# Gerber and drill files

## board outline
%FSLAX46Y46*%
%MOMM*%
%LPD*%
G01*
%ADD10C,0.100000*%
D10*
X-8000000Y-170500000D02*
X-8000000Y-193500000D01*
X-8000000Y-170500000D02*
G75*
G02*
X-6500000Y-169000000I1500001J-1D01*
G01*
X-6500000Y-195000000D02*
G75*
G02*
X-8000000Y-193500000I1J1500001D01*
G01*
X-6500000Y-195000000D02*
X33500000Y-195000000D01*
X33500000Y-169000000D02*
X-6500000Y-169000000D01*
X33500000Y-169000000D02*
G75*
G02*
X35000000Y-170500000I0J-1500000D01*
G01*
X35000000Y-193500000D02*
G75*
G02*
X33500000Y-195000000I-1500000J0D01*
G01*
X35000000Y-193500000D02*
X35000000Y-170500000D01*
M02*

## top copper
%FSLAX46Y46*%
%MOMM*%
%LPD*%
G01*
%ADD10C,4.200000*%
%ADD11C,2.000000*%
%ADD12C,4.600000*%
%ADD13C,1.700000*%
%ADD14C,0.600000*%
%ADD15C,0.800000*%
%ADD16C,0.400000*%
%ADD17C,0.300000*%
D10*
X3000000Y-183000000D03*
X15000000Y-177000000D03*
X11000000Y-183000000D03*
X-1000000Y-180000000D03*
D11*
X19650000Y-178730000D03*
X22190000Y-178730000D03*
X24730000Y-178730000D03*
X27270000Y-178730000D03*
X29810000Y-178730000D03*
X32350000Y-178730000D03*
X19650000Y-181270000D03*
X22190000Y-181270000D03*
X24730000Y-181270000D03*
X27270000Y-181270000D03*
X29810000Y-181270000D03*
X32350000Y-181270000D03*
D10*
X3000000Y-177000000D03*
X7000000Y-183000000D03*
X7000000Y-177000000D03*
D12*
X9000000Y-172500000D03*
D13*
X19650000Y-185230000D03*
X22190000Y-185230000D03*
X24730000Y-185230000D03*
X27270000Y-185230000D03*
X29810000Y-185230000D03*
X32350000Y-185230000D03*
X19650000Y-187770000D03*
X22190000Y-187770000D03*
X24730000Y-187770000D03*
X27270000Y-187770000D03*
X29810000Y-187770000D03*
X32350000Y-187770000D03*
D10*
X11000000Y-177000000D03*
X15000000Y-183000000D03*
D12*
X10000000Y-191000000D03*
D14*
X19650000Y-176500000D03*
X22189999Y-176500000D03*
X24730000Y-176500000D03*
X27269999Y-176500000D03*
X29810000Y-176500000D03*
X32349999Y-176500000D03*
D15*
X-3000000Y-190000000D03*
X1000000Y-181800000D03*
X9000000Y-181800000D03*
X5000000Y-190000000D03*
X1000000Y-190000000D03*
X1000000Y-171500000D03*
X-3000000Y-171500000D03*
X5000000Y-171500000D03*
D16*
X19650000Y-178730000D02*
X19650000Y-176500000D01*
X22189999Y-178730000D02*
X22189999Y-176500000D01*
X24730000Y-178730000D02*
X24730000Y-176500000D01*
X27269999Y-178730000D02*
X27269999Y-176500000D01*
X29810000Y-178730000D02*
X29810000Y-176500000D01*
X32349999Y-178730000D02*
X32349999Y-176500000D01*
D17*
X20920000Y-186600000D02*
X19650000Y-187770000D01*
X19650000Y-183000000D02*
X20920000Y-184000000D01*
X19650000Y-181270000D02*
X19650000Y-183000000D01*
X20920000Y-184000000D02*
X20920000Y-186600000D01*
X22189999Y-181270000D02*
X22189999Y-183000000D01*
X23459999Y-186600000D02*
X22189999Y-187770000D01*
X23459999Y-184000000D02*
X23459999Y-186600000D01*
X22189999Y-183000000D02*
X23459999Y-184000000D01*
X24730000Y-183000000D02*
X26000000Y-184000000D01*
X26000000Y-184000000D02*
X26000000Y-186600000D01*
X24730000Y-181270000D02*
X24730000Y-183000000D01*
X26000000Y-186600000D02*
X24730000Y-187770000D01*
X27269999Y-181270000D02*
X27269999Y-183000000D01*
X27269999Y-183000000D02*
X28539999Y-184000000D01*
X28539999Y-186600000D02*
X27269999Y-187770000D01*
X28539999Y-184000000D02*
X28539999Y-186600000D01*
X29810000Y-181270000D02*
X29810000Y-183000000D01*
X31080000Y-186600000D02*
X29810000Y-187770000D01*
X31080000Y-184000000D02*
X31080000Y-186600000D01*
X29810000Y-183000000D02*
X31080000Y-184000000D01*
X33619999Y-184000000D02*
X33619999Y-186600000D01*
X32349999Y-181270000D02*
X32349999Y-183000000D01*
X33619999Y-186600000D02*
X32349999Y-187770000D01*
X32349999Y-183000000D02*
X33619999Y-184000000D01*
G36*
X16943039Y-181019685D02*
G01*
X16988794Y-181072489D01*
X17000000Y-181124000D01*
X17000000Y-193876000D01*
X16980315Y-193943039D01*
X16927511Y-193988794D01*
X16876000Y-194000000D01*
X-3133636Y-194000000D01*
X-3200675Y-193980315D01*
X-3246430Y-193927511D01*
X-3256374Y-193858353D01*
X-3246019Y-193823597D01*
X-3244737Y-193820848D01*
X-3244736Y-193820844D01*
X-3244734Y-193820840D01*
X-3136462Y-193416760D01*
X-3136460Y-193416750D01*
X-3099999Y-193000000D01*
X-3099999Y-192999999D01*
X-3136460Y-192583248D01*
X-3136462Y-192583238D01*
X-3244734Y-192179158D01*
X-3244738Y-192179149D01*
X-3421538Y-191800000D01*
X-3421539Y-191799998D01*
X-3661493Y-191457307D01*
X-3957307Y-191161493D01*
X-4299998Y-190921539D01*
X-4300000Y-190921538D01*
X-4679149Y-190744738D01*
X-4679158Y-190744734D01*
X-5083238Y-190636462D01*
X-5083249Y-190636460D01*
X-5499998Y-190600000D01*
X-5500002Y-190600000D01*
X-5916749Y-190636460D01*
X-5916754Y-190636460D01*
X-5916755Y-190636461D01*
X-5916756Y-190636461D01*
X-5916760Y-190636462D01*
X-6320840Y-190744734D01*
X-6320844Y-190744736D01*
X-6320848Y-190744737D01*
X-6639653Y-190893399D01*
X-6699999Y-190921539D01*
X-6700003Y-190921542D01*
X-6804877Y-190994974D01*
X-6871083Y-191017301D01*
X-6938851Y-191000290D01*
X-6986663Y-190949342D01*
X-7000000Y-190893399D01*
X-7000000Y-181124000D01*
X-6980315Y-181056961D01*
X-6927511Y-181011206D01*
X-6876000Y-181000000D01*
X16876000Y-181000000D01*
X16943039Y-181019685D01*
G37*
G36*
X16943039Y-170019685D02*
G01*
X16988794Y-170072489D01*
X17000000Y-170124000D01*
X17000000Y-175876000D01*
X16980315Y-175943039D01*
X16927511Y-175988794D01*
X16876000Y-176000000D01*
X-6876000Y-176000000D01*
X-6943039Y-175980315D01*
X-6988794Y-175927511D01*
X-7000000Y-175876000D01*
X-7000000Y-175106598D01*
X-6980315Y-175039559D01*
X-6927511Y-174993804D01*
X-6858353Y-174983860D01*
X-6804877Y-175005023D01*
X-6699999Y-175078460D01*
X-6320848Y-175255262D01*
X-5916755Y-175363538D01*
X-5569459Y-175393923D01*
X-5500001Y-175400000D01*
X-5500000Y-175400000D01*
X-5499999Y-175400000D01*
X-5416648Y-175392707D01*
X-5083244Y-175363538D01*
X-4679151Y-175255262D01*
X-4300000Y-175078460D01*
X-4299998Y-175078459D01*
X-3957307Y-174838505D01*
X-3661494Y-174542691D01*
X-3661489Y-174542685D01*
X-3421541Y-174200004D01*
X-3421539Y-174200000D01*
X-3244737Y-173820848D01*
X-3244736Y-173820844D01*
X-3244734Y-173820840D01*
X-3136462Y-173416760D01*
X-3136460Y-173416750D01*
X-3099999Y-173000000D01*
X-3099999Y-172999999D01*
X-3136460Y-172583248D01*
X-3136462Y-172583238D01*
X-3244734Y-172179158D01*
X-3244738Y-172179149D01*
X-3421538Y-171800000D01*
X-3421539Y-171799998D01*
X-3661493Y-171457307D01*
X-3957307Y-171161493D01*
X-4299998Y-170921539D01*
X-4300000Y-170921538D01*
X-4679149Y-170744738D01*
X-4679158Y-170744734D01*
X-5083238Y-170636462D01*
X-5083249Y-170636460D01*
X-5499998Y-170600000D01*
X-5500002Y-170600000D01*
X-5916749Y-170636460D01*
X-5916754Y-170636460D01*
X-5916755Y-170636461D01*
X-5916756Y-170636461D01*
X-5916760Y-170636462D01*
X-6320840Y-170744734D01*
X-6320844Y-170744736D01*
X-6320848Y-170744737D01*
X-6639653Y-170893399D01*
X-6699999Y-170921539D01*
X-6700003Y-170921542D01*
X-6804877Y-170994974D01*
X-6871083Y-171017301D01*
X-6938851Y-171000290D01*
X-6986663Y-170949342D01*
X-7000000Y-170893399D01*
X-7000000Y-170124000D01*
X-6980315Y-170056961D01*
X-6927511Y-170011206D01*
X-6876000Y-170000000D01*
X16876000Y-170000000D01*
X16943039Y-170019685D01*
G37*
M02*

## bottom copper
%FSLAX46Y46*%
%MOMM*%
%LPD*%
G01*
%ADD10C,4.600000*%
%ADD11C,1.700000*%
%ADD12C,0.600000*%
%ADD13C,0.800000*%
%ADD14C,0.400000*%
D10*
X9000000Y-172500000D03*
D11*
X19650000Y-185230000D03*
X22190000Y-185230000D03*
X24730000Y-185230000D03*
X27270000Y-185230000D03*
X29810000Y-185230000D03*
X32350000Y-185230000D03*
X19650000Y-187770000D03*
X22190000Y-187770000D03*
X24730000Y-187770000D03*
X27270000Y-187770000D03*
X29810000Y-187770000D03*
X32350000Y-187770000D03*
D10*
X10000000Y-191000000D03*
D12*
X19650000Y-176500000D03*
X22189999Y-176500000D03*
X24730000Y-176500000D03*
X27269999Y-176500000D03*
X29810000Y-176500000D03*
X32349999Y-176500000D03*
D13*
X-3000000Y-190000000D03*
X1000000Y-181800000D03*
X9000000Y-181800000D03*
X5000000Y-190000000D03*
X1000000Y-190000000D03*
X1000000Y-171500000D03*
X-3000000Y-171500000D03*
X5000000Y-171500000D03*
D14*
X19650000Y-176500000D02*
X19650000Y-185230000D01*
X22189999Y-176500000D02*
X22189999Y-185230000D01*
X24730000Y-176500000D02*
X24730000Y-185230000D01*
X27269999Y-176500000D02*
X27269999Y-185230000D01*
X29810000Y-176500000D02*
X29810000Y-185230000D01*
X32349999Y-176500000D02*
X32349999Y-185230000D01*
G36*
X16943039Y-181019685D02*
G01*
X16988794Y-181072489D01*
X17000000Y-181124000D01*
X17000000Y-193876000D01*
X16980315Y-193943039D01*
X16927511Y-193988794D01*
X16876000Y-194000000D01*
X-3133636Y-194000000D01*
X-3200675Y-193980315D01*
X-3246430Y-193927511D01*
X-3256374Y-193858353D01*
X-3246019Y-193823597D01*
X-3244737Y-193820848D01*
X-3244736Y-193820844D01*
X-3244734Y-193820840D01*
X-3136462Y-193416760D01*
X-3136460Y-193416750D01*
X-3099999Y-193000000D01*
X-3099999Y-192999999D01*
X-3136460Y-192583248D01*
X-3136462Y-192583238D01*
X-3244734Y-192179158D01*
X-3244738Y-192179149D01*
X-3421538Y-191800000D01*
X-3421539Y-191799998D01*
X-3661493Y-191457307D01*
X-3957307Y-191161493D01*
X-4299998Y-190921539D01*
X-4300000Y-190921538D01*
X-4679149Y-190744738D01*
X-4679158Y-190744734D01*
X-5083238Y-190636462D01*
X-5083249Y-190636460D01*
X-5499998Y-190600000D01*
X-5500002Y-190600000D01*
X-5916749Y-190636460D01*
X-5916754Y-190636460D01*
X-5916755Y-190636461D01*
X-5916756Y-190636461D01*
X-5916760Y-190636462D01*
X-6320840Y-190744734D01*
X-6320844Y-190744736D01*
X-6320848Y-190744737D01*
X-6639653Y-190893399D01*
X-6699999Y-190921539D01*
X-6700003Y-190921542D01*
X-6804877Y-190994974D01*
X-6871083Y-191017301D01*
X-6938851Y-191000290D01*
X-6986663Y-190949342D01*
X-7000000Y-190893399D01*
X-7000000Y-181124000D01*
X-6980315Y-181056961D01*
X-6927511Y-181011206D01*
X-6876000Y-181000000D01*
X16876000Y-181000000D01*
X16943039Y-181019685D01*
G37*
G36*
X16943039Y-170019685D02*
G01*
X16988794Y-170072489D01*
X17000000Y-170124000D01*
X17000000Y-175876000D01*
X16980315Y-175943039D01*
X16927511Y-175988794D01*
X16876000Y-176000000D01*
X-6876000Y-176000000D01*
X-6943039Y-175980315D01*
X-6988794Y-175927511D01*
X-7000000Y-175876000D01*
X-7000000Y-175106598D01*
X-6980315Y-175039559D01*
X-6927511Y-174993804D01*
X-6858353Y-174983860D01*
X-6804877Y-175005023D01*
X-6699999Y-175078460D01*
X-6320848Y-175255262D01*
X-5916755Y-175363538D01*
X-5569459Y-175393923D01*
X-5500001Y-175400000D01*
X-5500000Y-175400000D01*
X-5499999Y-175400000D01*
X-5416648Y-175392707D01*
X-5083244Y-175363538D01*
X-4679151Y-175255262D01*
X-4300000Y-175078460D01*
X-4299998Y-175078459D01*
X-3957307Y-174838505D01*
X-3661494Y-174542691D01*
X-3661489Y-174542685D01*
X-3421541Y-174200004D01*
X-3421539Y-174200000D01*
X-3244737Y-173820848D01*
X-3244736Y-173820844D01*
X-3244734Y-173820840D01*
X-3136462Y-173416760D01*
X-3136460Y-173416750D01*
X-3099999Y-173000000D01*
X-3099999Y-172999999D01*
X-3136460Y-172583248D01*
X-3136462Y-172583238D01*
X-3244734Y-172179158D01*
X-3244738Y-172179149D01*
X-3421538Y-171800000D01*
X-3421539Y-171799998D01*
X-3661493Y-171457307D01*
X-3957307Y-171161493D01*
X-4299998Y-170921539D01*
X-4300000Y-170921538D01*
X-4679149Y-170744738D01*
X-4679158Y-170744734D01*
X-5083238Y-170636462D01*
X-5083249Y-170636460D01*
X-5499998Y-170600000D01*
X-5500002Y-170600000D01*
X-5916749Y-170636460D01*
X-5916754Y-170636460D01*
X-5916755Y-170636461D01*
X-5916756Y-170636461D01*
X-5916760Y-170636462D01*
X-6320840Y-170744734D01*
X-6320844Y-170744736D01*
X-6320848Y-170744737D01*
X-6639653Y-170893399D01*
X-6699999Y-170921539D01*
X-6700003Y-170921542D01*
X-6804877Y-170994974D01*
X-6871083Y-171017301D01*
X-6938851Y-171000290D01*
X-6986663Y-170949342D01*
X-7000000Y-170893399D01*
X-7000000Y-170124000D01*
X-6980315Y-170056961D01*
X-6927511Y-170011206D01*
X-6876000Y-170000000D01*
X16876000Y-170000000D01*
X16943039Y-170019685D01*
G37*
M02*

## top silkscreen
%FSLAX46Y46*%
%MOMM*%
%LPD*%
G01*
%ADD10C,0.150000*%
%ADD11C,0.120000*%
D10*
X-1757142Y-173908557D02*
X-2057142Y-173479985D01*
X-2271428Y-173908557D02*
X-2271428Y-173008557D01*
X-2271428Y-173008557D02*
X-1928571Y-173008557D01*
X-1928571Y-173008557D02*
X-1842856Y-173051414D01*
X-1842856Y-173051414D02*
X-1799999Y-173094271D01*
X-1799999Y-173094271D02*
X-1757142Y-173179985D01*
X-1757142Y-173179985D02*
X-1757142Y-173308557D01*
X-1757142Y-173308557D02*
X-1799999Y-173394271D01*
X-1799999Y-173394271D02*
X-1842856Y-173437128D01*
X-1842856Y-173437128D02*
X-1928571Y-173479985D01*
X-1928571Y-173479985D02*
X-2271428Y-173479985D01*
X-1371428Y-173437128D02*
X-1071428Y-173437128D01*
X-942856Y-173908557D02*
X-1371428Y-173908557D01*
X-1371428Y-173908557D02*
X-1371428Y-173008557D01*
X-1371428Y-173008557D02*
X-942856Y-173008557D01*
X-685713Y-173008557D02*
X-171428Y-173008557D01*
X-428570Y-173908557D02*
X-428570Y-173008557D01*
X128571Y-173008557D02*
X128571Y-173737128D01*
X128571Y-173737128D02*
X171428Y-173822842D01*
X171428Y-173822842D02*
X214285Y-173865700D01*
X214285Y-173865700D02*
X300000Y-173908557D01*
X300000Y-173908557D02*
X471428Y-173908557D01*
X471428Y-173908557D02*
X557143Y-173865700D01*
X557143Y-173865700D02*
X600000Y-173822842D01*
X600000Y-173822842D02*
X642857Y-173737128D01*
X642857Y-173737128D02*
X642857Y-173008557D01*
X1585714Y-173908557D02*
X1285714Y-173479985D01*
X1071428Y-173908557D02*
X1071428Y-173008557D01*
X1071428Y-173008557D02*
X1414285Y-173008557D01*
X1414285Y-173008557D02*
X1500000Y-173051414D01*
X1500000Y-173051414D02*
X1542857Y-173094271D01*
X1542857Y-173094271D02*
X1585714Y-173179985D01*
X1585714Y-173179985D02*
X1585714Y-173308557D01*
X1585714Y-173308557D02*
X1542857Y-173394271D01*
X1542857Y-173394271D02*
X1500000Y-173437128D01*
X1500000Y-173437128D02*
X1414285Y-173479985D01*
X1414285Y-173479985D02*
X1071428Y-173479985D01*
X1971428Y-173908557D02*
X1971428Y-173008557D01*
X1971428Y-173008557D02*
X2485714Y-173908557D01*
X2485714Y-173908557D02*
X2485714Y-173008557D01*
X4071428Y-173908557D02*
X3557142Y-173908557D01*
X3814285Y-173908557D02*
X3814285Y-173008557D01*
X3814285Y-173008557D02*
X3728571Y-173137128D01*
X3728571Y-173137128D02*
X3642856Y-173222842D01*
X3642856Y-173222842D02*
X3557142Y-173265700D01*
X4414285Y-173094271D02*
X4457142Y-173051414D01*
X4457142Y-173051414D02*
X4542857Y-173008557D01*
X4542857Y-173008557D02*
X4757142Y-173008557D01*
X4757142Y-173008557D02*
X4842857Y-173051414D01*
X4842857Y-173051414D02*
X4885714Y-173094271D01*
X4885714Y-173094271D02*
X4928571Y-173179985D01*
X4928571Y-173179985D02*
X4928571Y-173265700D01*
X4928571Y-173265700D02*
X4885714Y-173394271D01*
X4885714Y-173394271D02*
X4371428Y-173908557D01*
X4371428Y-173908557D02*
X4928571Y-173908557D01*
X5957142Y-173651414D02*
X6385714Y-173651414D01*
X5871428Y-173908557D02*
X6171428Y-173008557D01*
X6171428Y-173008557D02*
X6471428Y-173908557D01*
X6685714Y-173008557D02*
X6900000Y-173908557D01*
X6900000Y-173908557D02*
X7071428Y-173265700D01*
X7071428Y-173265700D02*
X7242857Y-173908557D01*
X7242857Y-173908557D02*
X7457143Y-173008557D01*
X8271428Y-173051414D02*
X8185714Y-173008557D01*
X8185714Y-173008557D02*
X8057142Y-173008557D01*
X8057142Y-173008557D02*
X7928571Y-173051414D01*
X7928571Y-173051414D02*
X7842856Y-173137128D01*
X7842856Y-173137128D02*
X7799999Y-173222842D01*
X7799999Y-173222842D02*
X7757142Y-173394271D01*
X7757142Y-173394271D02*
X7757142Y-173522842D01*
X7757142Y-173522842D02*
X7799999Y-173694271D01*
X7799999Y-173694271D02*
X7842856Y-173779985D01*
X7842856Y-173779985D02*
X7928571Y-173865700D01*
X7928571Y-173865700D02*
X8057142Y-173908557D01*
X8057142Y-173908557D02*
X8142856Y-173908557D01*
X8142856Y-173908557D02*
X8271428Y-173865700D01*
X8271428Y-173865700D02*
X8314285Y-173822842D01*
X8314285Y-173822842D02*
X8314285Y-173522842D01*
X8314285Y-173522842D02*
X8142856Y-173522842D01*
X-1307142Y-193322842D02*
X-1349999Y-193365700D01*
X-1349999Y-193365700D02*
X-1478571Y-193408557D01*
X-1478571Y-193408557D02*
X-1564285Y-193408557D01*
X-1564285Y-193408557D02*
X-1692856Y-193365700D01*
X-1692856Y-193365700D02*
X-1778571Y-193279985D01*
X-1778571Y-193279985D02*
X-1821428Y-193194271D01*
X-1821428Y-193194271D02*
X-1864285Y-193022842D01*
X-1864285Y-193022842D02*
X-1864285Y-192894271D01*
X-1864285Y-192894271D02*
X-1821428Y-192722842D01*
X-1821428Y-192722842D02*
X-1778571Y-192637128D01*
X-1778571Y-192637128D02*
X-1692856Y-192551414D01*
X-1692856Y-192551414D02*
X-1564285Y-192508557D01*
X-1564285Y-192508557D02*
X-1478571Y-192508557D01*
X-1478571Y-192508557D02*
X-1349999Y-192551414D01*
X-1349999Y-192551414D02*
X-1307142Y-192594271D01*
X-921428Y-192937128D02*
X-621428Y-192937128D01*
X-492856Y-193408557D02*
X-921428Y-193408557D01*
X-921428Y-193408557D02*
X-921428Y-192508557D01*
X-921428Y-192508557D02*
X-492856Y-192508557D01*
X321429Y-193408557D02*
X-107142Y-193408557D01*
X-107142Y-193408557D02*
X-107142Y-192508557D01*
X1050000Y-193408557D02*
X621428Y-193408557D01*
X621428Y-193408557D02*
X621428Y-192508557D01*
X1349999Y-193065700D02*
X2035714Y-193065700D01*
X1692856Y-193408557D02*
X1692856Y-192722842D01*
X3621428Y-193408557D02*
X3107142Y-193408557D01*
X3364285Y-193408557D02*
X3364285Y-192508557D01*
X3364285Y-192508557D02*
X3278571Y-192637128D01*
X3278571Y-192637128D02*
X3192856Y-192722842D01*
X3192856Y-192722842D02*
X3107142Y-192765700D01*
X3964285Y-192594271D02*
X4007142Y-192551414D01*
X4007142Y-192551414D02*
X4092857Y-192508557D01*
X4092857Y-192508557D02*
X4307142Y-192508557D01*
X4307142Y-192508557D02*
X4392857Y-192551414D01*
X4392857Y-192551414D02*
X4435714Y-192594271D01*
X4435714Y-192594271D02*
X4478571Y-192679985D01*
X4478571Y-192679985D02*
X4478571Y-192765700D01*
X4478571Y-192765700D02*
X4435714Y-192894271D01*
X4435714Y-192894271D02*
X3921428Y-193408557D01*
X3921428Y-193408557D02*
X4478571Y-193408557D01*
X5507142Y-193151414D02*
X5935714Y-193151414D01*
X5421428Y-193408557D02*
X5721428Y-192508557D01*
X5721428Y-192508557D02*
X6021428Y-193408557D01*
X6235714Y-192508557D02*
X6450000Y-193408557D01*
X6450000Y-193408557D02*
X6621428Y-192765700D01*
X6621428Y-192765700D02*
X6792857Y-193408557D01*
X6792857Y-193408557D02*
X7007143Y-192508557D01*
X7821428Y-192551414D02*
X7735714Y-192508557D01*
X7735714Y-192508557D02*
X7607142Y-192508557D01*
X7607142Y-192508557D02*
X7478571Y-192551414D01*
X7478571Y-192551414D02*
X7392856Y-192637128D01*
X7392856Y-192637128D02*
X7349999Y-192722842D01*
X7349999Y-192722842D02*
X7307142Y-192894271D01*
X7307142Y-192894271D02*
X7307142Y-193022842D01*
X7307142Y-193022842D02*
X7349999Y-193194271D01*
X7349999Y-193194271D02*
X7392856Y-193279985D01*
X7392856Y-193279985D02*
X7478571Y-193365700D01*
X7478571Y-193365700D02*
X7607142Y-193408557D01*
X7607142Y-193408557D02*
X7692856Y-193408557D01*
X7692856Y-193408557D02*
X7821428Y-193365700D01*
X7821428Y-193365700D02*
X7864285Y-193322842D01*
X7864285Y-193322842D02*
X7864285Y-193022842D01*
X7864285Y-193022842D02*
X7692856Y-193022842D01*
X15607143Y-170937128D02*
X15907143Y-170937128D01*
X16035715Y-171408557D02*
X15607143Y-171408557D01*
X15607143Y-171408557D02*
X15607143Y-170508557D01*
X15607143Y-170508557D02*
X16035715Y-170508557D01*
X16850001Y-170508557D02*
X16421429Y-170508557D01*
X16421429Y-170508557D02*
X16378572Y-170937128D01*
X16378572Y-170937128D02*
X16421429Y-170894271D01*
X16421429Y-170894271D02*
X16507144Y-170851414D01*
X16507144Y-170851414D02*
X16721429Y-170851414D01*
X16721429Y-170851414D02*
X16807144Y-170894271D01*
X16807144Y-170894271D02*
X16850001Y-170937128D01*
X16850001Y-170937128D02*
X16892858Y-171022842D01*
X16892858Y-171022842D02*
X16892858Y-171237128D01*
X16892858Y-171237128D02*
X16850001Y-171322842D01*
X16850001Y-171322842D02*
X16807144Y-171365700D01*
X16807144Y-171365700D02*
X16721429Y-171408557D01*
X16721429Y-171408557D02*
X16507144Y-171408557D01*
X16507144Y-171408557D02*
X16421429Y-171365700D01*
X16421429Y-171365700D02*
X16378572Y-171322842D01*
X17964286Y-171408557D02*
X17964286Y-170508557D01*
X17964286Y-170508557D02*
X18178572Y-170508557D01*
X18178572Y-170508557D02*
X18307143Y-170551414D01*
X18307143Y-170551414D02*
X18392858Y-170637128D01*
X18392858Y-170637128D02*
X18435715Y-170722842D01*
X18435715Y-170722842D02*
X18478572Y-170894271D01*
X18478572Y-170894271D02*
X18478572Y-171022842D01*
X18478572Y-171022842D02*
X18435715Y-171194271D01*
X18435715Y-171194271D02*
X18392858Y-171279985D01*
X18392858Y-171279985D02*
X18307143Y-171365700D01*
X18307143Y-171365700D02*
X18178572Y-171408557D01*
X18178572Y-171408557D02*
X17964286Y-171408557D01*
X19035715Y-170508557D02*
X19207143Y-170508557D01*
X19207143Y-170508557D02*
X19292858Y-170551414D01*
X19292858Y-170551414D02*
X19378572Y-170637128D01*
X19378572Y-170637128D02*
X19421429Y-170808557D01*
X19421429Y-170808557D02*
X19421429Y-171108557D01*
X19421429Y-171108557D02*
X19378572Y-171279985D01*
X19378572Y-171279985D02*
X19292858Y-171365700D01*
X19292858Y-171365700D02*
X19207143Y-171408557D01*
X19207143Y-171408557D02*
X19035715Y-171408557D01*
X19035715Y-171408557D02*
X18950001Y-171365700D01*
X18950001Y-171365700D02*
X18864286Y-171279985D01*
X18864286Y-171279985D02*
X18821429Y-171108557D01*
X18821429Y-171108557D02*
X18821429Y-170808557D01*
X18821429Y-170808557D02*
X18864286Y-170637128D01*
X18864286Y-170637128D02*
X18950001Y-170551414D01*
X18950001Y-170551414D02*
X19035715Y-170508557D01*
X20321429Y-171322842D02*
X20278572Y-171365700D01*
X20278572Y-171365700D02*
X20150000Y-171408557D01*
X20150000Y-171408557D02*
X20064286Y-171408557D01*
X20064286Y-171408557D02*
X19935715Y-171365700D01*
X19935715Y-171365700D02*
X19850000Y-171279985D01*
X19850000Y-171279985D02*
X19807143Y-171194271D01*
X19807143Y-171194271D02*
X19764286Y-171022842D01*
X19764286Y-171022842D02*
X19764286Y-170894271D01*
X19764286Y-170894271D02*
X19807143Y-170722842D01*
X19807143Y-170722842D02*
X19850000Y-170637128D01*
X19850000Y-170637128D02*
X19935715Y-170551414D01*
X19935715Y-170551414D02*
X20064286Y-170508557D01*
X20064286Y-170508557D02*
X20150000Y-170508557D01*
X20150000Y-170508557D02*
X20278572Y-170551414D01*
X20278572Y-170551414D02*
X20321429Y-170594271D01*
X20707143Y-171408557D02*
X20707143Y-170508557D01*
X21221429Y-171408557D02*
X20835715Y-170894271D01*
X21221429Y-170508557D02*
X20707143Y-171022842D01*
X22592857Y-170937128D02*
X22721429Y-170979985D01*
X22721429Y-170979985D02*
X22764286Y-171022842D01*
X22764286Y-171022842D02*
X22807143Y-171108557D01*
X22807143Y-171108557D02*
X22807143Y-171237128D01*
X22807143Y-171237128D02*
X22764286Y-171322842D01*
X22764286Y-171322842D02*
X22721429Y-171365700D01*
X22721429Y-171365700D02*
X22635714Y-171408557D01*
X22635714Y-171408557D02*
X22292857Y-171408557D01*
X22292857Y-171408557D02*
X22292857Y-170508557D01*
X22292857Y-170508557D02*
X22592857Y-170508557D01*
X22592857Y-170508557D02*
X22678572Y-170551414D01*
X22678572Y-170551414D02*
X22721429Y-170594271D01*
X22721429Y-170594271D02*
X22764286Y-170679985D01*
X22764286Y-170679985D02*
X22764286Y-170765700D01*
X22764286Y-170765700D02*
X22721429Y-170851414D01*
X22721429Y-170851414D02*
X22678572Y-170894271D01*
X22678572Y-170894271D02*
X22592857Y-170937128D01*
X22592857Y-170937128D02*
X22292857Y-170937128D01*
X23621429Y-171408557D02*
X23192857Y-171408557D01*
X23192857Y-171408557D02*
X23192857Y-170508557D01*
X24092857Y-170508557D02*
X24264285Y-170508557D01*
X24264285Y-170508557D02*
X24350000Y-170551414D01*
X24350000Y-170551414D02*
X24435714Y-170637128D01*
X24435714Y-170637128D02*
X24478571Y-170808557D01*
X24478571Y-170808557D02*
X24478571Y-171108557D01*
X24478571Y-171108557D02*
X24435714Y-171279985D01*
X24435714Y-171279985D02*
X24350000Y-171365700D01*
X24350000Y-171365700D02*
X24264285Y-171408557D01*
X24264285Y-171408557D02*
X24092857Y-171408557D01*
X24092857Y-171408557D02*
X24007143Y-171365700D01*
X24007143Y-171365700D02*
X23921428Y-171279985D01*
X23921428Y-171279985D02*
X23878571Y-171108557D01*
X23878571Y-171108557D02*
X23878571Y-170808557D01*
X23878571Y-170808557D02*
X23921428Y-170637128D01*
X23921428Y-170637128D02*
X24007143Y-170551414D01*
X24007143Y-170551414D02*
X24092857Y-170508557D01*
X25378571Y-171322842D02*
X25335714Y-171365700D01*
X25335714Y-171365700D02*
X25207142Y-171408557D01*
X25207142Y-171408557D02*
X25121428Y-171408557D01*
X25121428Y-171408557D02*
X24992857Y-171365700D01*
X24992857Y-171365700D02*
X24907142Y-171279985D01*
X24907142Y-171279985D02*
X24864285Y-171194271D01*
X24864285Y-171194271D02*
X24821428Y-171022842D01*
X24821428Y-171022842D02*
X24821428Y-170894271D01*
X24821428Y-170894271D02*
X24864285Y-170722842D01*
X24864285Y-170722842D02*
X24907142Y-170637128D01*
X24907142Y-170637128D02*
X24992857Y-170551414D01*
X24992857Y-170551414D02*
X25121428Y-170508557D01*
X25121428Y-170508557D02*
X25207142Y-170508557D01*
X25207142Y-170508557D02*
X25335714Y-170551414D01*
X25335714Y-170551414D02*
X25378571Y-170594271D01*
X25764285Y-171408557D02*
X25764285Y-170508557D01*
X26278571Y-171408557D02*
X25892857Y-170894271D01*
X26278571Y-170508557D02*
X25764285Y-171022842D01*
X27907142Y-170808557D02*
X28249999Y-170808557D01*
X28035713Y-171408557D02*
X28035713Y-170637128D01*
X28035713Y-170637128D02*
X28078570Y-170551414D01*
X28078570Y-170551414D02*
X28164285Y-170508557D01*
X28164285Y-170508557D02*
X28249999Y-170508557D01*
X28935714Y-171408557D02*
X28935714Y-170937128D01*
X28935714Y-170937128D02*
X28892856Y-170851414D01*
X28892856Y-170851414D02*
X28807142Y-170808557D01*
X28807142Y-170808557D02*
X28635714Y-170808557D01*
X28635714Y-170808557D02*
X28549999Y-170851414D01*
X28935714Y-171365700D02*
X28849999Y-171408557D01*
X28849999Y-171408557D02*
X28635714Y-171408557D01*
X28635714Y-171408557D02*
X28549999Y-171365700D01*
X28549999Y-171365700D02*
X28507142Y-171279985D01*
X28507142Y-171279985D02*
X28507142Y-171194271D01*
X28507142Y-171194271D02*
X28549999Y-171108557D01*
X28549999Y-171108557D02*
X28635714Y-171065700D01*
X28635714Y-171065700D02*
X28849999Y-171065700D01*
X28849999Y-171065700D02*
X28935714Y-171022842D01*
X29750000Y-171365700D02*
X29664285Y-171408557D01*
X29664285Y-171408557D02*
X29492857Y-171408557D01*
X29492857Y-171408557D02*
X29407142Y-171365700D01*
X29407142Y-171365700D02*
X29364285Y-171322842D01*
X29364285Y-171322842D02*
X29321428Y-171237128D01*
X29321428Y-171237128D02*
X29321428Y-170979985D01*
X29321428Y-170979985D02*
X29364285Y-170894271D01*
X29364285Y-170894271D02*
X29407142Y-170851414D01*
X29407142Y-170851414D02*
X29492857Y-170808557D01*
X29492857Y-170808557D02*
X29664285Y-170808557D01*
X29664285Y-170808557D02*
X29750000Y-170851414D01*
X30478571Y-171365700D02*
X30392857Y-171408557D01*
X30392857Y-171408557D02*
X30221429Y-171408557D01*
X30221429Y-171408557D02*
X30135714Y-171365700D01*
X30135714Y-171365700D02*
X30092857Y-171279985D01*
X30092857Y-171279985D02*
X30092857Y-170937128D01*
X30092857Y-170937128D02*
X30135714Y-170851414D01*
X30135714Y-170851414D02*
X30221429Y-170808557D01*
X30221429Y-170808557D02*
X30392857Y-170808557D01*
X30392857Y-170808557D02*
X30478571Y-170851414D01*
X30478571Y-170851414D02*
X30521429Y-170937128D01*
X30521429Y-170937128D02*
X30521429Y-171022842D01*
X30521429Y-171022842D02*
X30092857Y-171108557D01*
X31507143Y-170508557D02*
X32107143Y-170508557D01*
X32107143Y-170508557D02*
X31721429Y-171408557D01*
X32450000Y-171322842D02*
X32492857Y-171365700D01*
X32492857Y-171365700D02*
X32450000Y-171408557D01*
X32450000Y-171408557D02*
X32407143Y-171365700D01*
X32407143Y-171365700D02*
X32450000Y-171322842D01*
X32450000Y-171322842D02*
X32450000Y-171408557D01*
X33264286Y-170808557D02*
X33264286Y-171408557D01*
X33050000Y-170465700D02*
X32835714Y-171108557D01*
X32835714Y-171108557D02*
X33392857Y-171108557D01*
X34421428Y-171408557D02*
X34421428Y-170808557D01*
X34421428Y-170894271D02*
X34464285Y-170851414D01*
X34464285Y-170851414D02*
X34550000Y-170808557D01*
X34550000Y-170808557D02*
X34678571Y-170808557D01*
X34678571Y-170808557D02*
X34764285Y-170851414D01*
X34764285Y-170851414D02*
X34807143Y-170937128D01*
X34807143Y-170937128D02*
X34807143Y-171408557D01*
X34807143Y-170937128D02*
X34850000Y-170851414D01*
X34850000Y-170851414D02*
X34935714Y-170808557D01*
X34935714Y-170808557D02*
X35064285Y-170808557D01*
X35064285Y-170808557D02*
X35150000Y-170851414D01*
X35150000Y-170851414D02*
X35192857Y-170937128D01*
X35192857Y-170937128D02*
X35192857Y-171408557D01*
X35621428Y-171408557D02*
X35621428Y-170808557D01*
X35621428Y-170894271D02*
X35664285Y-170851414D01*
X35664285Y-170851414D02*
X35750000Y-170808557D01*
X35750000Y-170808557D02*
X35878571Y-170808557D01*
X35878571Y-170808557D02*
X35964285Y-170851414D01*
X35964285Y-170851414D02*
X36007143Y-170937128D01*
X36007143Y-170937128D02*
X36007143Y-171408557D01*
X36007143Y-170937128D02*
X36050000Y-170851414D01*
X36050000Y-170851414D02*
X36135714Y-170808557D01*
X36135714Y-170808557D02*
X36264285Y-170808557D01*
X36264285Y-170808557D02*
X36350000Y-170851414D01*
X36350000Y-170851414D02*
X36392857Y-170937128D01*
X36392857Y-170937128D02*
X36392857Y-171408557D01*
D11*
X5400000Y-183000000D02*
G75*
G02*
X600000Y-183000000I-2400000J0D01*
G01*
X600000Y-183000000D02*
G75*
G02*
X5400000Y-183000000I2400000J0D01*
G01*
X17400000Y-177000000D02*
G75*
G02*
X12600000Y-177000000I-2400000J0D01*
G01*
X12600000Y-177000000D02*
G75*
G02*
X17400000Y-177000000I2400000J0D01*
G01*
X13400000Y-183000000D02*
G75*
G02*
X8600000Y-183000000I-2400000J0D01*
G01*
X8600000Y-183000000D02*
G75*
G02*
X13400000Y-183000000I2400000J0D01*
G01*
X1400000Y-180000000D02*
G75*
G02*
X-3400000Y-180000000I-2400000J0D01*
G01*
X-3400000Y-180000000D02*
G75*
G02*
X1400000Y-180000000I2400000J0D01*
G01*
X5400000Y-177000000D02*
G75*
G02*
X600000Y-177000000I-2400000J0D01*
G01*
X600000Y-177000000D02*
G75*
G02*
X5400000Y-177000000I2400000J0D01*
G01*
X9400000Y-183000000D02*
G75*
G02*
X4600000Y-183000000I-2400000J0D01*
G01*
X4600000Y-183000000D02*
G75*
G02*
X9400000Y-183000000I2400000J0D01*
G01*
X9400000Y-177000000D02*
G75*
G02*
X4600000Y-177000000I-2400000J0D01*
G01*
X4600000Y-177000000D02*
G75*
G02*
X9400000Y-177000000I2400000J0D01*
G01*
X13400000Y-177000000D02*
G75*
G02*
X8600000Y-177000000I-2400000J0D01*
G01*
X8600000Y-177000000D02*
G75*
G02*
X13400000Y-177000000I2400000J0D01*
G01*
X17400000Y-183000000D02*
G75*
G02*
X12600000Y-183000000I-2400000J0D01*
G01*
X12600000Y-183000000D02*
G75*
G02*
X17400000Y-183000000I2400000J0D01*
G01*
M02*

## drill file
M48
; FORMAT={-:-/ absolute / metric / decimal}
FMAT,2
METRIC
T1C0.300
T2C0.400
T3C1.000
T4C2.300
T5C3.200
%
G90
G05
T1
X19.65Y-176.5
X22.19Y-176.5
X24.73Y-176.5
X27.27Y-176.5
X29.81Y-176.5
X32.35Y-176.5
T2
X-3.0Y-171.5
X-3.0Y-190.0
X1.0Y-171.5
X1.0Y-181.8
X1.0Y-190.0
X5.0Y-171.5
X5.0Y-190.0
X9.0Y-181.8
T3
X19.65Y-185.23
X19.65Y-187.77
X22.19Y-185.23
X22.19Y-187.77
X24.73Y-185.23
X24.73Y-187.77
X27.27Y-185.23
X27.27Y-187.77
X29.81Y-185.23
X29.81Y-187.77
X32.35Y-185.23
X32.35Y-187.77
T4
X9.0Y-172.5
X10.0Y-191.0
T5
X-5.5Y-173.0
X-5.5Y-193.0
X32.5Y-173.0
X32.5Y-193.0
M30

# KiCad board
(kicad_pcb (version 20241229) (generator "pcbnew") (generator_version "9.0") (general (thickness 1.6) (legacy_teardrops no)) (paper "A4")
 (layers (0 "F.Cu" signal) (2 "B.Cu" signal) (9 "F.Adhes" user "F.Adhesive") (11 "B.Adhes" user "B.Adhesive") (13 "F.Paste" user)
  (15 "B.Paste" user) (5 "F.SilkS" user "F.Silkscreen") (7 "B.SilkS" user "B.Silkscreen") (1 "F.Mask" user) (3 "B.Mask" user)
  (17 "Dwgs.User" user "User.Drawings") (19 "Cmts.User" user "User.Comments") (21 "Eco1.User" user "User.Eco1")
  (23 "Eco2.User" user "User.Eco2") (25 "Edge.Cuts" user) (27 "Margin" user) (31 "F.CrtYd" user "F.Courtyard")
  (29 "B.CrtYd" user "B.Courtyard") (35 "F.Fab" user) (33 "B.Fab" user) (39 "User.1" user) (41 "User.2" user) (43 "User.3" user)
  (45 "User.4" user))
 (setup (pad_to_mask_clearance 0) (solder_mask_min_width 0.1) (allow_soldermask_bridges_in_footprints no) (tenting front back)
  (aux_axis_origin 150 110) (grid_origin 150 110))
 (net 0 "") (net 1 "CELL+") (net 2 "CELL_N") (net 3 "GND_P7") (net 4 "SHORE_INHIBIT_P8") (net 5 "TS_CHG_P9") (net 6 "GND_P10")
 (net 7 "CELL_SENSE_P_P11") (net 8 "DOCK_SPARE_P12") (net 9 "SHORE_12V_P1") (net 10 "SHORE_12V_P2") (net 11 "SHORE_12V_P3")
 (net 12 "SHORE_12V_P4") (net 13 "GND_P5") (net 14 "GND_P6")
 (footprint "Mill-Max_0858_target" (layer "F.Cu") (at 3 183)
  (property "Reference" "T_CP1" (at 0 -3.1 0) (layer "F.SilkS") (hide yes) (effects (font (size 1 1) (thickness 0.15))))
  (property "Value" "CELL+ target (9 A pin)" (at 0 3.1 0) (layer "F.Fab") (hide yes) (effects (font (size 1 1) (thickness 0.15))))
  (fp_circle (center 0 0) (end 2.4 0) (stroke (width 0.12) (type solid)) (fill no) (layer "F.SilkS"))
  (pad "1" smd circle (at 0 0) (size 4.2 4.2) (layers "F.Cu" "F.Mask") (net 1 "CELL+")))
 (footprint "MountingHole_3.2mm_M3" (layer "F.Cu") (at -5.5 173)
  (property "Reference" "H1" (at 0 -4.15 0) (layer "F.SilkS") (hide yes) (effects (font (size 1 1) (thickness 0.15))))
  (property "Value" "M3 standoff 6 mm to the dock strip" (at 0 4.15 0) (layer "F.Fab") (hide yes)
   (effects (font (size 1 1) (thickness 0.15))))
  (pad "" np_thru_hole circle (at 0 0) (size 3.2 3.2) (drill 3.2) (layers "*.Cu" "*.Mask")))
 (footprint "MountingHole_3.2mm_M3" (layer "F.Cu") (at 32.5 173)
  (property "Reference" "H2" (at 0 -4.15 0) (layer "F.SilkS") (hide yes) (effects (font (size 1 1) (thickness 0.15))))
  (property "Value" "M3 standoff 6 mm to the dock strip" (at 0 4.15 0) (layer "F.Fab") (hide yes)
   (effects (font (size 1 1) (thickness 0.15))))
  (pad "" np_thru_hole circle (at 0 0) (size 3.2 3.2) (drill 3.2) (layers "*.Cu" "*.Mask")))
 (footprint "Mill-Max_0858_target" (layer "F.Cu") (at 15 177)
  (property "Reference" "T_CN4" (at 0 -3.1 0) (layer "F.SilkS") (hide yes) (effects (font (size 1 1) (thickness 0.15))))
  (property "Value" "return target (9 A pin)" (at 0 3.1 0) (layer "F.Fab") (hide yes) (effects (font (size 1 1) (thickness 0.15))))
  (fp_circle (center 0 0) (end 2.4 0) (stroke (width 0.12) (type solid)) (fill no) (layer "F.SilkS"))
  (pad "1" smd circle (at 0 0) (size 4.2 4.2) (layers "F.Cu" "F.Mask") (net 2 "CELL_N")))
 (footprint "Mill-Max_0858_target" (layer "F.Cu") (at 11 183)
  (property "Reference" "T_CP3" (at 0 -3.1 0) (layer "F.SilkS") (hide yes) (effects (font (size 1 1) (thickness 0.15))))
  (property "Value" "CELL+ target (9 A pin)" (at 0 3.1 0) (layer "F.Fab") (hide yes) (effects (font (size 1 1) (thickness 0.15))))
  (fp_circle (center 0 0) (end 2.4 0) (stroke (width 0.12) (type solid)) (fill no) (layer "F.SilkS"))
  (pad "1" smd circle (at 0 0) (size 4.2 4.2) (layers "F.Cu" "F.Mask") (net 1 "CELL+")))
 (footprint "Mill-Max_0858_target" (layer "F.Cu") (at -1 180)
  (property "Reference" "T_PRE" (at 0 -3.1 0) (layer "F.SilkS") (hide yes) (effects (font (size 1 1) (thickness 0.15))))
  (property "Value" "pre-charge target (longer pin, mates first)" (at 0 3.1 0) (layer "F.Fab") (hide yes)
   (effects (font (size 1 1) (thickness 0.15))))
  (fp_circle (center 0 0) (end 2.4 0) (stroke (width 0.12) (type solid)) (fill no) (layer "F.SilkS"))
  (pad "1" smd circle (at 0 0) (size 4.2 4.2) (layers "F.Cu" "F.Mask") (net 1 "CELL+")))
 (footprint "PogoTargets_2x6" (layer "F.Cu") (at 26 180)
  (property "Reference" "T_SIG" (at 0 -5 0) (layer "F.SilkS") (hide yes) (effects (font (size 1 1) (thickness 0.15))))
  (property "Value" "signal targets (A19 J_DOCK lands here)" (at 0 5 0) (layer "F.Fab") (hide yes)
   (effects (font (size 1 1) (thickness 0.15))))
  (pad "1" smd circle (at -6.35 -1.27) (size 2 2) (layers "F.Cu" "F.Mask") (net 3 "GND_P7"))
  (pad "2" smd circle (at -3.81 -1.27) (size 2 2) (layers "F.Cu" "F.Mask") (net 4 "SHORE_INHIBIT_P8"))
  (pad "3" smd circle (at -1.27 -1.27) (size 2 2) (layers "F.Cu" "F.Mask") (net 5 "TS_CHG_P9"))
  (pad "4" smd circle (at 1.27 -1.27) (size 2 2) (layers "F.Cu" "F.Mask") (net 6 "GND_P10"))
  (pad "5" smd circle (at 3.81 -1.27) (size 2 2) (layers "F.Cu" "F.Mask") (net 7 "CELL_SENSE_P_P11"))
  (pad "6" smd circle (at 6.35 -1.27) (size 2 2) (layers "F.Cu" "F.Mask") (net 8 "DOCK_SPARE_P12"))
  (pad "7" smd circle (at -6.35 1.27) (size 2 2) (layers "F.Cu" "F.Mask") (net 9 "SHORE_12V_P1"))
  (pad "8" smd circle (at -3.81 1.27) (size 2 2) (layers "F.Cu" "F.Mask") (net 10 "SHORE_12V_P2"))
  (pad "9" smd circle (at -1.27 1.27) (size 2 2) (layers "F.Cu" "F.Mask") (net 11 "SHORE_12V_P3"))
  (pad "10" smd circle (at 1.27 1.27) (size 2 2) (layers "F.Cu" "F.Mask") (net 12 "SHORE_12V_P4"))
  (pad "11" smd circle (at 3.81 1.27) (size 2 2) (layers "F.Cu" "F.Mask") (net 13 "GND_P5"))
  (pad "12" smd circle (at 6.35 1.27) (size 2 2) (layers "F.Cu" "F.Mask") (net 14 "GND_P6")))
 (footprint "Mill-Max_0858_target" (layer "F.Cu") (at 3 177)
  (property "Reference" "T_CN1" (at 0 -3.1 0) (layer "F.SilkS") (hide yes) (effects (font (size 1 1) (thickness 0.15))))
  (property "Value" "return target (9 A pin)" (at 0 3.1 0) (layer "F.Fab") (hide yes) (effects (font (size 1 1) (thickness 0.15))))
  (fp_circle (center 0 0) (end 2.4 0) (stroke (width 0.12) (type solid)) (fill no) (layer "F.SilkS"))
  (pad "1" smd circle (at 0 0) (size 4.2 4.2) (layers "F.Cu" "F.Mask") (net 2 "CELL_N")))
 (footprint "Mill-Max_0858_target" (layer "F.Cu") (at 7 183)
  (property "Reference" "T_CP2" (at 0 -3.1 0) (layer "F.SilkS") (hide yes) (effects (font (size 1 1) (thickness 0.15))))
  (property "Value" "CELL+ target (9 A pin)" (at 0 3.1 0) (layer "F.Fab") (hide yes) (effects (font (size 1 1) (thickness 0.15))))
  (fp_circle (center 0 0) (end 2.4 0) (stroke (width 0.12) (type solid)) (fill no) (layer "F.SilkS"))
  (pad "1" smd circle (at 0 0) (size 4.2 4.2) (layers "F.Cu" "F.Mask") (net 1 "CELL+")))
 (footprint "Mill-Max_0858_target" (layer "F.Cu") (at 7 177)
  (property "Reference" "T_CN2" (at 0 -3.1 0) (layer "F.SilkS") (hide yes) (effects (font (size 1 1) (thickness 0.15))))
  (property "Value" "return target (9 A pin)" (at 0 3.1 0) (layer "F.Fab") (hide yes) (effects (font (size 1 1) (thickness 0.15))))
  (fp_circle (center 0 0) (end 2.4 0) (stroke (width 0.12) (type solid)) (fill no) (layer "F.SilkS"))
  (pad "1" smd circle (at 0 0) (size 4.2 4.2) (layers "F.Cu" "F.Mask") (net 2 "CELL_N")))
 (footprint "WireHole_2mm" (layer "F.Cu") (at 9 172.5)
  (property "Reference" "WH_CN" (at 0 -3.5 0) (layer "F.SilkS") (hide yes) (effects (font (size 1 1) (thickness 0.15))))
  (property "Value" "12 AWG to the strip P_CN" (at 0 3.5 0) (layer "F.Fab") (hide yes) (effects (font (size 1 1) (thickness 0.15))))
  (pad "1" thru_hole circle (at 0 0) (size 4.6 4.6) (drill 2.3) (layers "*.Cu" "*.Mask") (remove_unused_layers no) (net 2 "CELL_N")))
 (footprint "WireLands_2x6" (layer "F.Cu") (at 26 186.5)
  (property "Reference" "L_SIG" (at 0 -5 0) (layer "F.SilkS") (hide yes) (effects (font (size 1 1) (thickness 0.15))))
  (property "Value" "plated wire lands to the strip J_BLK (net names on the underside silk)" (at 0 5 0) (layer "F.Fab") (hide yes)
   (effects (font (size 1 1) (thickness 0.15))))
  (pad "1" thru_hole circle (at -6.35 -1.27) (size 1.7 1.7) (drill 1) (layers "*.Cu" "*.Mask") (remove_unused_layers no) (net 3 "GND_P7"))
  (pad "2" thru_hole circle (at -3.81 -1.27) (size 1.7 1.7) (drill 1) (layers "*.Cu" "*.Mask") (remove_unused_layers no)
   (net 4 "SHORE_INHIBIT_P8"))
  (pad "3" thru_hole circle (at -1.27 -1.27) (size 1.7 1.7) (drill 1) (layers "*.Cu" "*.Mask") (remove_unused_layers no) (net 5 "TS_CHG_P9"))
  (pad "4" thru_hole circle (at 1.27 -1.27) (size 1.7 1.7) (drill 1) (layers "*.Cu" "*.Mask") (remove_unused_layers no) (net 6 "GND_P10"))
  (pad "5" thru_hole circle (at 3.81 -1.27) (size 1.7 1.7) (drill 1) (layers "*.Cu" "*.Mask") (remove_unused_layers no)
   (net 7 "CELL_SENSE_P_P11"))
  (pad "6" thru_hole circle (at 6.35 -1.27) (size 1.7 1.7) (drill 1) (layers "*.Cu" "*.Mask") (remove_unused_layers no)
   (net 8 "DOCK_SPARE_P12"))
  (pad "7" thru_hole circle (at -6.35 1.27) (size 1.7 1.7) (drill 1) (layers "*.Cu" "*.Mask") (remove_unused_layers no)
   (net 9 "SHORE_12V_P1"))
  (pad "8" thru_hole circle (at -3.81 1.27) (size 1.7 1.7) (drill 1) (layers "*.Cu" "*.Mask") (remove_unused_layers no)
   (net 10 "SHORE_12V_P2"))
  (pad "9" thru_hole circle (at -1.27 1.27) (size 1.7 1.7) (drill 1) (layers "*.Cu" "*.Mask") (remove_unused_layers no)
   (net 11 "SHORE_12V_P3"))
  (pad "10" thru_hole circle (at 1.27 1.27) (size 1.7 1.7) (drill 1) (layers "*.Cu" "*.Mask") (remove_unused_layers no)
   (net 12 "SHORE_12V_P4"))
  (pad "11" thru_hole circle (at 3.81 1.27) (size 1.7 1.7) (drill 1) (layers "*.Cu" "*.Mask") (remove_unused_layers no) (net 13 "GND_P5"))
  (pad "12" thru_hole circle (at 6.35 1.27) (size 1.7 1.7) (drill 1) (layers "*.Cu" "*.Mask") (remove_unused_layers no) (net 14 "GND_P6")))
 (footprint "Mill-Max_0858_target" (layer "F.Cu") (at 11 177)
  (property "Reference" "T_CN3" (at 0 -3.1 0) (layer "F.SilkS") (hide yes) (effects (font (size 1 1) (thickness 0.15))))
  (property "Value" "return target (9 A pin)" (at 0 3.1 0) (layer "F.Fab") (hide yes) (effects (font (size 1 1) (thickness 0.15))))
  (fp_circle (center 0 0) (end 2.4 0) (stroke (width 0.12) (type solid)) (fill no) (layer "F.SilkS"))
  (pad "1" smd circle (at 0 0) (size 4.2 4.2) (layers "F.Cu" "F.Mask") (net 2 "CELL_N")))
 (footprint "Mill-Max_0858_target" (layer "F.Cu") (at 15 183)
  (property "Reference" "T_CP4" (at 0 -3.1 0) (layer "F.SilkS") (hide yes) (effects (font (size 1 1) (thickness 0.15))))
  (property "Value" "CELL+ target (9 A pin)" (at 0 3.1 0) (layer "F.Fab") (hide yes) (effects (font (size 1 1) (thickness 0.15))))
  (fp_circle (center 0 0) (end 2.4 0) (stroke (width 0.12) (type solid)) (fill no) (layer "F.SilkS"))
  (pad "1" smd circle (at 0 0) (size 4.2 4.2) (layers "F.Cu" "F.Mask") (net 1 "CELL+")))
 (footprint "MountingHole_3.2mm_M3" (layer "F.Cu") (at -5.5 193)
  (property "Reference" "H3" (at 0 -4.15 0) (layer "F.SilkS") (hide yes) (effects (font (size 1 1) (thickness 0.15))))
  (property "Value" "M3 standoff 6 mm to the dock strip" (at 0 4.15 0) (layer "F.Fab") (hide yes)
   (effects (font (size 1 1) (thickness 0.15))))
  (pad "" np_thru_hole circle (at 0 0) (size 3.2 3.2) (drill 3.2) (layers "*.Cu" "*.Mask")))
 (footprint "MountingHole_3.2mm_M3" (layer "F.Cu") (at 32.5 193)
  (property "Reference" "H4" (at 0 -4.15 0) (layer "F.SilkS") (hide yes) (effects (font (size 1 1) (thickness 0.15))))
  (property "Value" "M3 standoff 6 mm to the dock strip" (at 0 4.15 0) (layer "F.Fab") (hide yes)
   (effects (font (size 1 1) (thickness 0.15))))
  (pad "" np_thru_hole circle (at 0 0) (size 3.2 3.2) (drill 3.2) (layers "*.Cu" "*.Mask")))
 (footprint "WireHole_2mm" (layer "F.Cu") (at 10 191)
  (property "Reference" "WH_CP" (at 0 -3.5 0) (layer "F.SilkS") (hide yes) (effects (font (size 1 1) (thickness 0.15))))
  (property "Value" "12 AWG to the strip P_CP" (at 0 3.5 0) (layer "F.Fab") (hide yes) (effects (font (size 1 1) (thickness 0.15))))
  (pad "1" thru_hole circle (at 0 0) (size 4.6 4.6) (drill 2.3) (layers "*.Cu" "*.Mask") (remove_unused_layers no) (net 1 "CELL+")))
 (gr_line (start -8 170.5) (end -8 193.5) (stroke (width 0.1) (type default)) (layer "Edge.Cuts"))
 (gr_arc (start -8 170.5) (mid -7.56066 169.43934) (end -6.5 169) (stroke (width 0.1) (type default)) (layer "Edge.Cuts"))
 (gr_arc (start -6.5 195) (mid -7.56066 194.56066) (end -8 193.5) (stroke (width 0.1) (type default)) (layer "Edge.Cuts"))
 (gr_line (start -6.5 195) (end 33.5 195) (stroke (width 0.1) (type default)) (layer "Edge.Cuts"))
 (gr_line (start 33.5 169) (end -6.5 169) (stroke (width 0.1) (type default)) (layer "Edge.Cuts"))
 (gr_arc (start 33.5 169) (mid 34.56066 169.43934) (end 35 170.5) (stroke (width 0.1) (type default)) (layer "Edge.Cuts"))
 (gr_arc (start 35 193.5) (mid 34.56066 194.56066) (end 33.5 195) (stroke (width 0.1) (type default)) (layer "Edge.Cuts"))
 (gr_line (start 35 193.5) (end 35 170.5) (stroke (width 0.1) (type default)) (layer "Edge.Cuts"))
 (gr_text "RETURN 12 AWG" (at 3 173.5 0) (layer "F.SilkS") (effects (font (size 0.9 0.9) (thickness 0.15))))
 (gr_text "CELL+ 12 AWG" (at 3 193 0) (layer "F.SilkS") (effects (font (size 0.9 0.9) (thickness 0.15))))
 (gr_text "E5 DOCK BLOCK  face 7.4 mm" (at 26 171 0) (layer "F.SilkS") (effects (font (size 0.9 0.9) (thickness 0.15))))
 (segment (start 19.65 178.73) (end 19.65 176.5) (width 0.4) (layer "F.Cu") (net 3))
 (via (at 19.65 176.5) (size 0.6) (drill 0.3) (layers "F.Cu" "B.Cu") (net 3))
 (segment (start 19.65 176.5) (end 19.65 185.23) (width 0.4) (layer "B.Cu") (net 3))
 (segment (start 22.189999 178.73) (end 22.189999 176.5) (width 0.4) (layer "F.Cu") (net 4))
 (via (at 22.189999 176.5) (size 0.6) (drill 0.3) (layers "F.Cu" "B.Cu") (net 4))
 (segment (start 22.189999 176.5) (end 22.189999 185.23) (width 0.4) (layer "B.Cu") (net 4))
 (segment (start 24.73 178.73) (end 24.73 176.5) (width 0.4) (layer "F.Cu") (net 5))
 (via (at 24.73 176.5) (size 0.6) (drill 0.3) (layers "F.Cu" "B.Cu") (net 5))
 (segment (start 24.73 176.5) (end 24.73 185.23) (width 0.4) (layer "B.Cu") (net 5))
 (segment (start 27.269999 178.73) (end 27.269999 176.5) (width 0.4) (layer "F.Cu") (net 6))
 (via (at 27.269999 176.5) (size 0.6) (drill 0.3) (layers "F.Cu" "B.Cu") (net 6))
 (segment (start 27.269999 176.5) (end 27.269999 185.23) (width 0.4) (layer "B.Cu") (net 6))
 (segment (start 29.81 178.73) (end 29.81 176.5) (width 0.4) (layer "F.Cu") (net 7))
 (via (at 29.81 176.5) (size 0.6) (drill 0.3) (layers "F.Cu" "B.Cu") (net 7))
 (segment (start 29.81 176.5) (end 29.81 185.23) (width 0.4) (layer "B.Cu") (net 7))
 (segment (start 32.349999 178.73) (end 32.349999 176.5) (width 0.4) (layer "F.Cu") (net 8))
 (via (at 32.349999 176.5) (size 0.6) (drill 0.3) (layers "F.Cu" "B.Cu") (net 8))
 (segment (start 32.349999 176.5) (end 32.349999 185.23) (width 0.4) (layer "B.Cu") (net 8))
 (segment (start 20.92 186.6) (end 19.65 187.77) (width 0.3) (layer "F.Cu") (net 9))
 (segment (start 19.65 183) (end 20.92 184) (width 0.3) (layer "F.Cu") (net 9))
 (segment (start 19.65 181.27) (end 19.65 183) (width 0.3) (layer "F.Cu") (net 9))
 (segment (start 20.92 184) (end 20.92 186.6) (width 0.3) (layer "F.Cu") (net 9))
 (segment (start 22.189999 181.27) (end 22.189999 183) (width 0.3) (layer "F.Cu") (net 10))
 (segment (start 23.459999 186.6) (end 22.189999 187.77) (width 0.3) (layer "F.Cu") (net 10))
 (segment (start 23.459999 184) (end 23.459999 186.6) (width 0.3) (layer "F.Cu") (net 10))
 (segment (start 22.189999 183) (end 23.459999 184) (width 0.3) (layer "F.Cu") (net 10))
 (segment (start 24.73 183) (end 26 184) (width 0.3) (layer "F.Cu") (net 11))
 (segment (start 26 184) (end 26 186.6) (width 0.3) (layer "F.Cu") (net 11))
 (segment (start 24.73 181.27) (end 24.73 183) (width 0.3) (layer "F.Cu") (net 11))
 (segment (start 26 186.6) (end 24.73 187.77) (width 0.3) (layer "F.Cu") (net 11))
 (segment (start 27.269999 181.27) (end 27.269999 183) (width 0.3) (layer "F.Cu") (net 12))
 (segment (start 27.269999 183) (end 28.539999 184) (width 0.3) (layer "F.Cu") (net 12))
 (segment (start 28.539999 186.6) (end 27.269999 187.77) (width 0.3) (layer "F.Cu") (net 12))
 (segment (start 28.539999 184) (end 28.539999 186.6) (width 0.3) (layer "F.Cu") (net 12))
 (segment (start 29.81 181.27) (end 29.81 183) (width 0.3) (layer "F.Cu") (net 13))
 (segment (start 31.08 186.6) (end 29.81 187.77) (width 0.3) (layer "F.Cu") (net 13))
 (segment (start 31.08 184) (end 31.08 186.6) (width 0.3) (layer "F.Cu") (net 13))
 (segment (start 29.81 183) (end 31.08 184) (width 0.3) (layer "F.Cu") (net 13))
 (segment (start 33.619999 184) (end 33.619999 186.6) (width 0.3) (layer "F.Cu") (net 14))
 (segment (start 32.349999 181.27) (end 32.349999 183) (width 0.3) (layer "F.Cu") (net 14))
 (segment (start 33.619999 186.6) (end 32.349999 187.77) (width 0.3) (layer "F.Cu") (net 14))
 (segment (start 32.349999 183) (end 33.619999 184) (width 0.3) (layer "F.Cu") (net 14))
 (via (at -3 190) (size 0.8) (drill 0.4) (layers "F.Cu" "B.Cu") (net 1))
 (via (at 1 181.8) (size 0.8) (drill 0.4) (layers "F.Cu" "B.Cu") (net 1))
 (via (at 9 181.8) (size 0.8) (drill 0.4) (layers "F.Cu" "B.Cu") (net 1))
 (via (at 5 190) (size 0.8) (drill 0.4) (layers "F.Cu" "B.Cu") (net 1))
 (via (at 1 190) (size 0.8) (drill 0.4) (layers "F.Cu" "B.Cu") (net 1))
 (via (at 1 171.5) (size 0.8) (drill 0.4) (layers "F.Cu" "B.Cu") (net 2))
 (via (at -3 171.5) (size 0.8) (drill 0.4) (layers "F.Cu" "B.Cu") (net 2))
 (via (at 5 171.5) (size 0.8) (drill 0.4) (layers "F.Cu" "B.Cu") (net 2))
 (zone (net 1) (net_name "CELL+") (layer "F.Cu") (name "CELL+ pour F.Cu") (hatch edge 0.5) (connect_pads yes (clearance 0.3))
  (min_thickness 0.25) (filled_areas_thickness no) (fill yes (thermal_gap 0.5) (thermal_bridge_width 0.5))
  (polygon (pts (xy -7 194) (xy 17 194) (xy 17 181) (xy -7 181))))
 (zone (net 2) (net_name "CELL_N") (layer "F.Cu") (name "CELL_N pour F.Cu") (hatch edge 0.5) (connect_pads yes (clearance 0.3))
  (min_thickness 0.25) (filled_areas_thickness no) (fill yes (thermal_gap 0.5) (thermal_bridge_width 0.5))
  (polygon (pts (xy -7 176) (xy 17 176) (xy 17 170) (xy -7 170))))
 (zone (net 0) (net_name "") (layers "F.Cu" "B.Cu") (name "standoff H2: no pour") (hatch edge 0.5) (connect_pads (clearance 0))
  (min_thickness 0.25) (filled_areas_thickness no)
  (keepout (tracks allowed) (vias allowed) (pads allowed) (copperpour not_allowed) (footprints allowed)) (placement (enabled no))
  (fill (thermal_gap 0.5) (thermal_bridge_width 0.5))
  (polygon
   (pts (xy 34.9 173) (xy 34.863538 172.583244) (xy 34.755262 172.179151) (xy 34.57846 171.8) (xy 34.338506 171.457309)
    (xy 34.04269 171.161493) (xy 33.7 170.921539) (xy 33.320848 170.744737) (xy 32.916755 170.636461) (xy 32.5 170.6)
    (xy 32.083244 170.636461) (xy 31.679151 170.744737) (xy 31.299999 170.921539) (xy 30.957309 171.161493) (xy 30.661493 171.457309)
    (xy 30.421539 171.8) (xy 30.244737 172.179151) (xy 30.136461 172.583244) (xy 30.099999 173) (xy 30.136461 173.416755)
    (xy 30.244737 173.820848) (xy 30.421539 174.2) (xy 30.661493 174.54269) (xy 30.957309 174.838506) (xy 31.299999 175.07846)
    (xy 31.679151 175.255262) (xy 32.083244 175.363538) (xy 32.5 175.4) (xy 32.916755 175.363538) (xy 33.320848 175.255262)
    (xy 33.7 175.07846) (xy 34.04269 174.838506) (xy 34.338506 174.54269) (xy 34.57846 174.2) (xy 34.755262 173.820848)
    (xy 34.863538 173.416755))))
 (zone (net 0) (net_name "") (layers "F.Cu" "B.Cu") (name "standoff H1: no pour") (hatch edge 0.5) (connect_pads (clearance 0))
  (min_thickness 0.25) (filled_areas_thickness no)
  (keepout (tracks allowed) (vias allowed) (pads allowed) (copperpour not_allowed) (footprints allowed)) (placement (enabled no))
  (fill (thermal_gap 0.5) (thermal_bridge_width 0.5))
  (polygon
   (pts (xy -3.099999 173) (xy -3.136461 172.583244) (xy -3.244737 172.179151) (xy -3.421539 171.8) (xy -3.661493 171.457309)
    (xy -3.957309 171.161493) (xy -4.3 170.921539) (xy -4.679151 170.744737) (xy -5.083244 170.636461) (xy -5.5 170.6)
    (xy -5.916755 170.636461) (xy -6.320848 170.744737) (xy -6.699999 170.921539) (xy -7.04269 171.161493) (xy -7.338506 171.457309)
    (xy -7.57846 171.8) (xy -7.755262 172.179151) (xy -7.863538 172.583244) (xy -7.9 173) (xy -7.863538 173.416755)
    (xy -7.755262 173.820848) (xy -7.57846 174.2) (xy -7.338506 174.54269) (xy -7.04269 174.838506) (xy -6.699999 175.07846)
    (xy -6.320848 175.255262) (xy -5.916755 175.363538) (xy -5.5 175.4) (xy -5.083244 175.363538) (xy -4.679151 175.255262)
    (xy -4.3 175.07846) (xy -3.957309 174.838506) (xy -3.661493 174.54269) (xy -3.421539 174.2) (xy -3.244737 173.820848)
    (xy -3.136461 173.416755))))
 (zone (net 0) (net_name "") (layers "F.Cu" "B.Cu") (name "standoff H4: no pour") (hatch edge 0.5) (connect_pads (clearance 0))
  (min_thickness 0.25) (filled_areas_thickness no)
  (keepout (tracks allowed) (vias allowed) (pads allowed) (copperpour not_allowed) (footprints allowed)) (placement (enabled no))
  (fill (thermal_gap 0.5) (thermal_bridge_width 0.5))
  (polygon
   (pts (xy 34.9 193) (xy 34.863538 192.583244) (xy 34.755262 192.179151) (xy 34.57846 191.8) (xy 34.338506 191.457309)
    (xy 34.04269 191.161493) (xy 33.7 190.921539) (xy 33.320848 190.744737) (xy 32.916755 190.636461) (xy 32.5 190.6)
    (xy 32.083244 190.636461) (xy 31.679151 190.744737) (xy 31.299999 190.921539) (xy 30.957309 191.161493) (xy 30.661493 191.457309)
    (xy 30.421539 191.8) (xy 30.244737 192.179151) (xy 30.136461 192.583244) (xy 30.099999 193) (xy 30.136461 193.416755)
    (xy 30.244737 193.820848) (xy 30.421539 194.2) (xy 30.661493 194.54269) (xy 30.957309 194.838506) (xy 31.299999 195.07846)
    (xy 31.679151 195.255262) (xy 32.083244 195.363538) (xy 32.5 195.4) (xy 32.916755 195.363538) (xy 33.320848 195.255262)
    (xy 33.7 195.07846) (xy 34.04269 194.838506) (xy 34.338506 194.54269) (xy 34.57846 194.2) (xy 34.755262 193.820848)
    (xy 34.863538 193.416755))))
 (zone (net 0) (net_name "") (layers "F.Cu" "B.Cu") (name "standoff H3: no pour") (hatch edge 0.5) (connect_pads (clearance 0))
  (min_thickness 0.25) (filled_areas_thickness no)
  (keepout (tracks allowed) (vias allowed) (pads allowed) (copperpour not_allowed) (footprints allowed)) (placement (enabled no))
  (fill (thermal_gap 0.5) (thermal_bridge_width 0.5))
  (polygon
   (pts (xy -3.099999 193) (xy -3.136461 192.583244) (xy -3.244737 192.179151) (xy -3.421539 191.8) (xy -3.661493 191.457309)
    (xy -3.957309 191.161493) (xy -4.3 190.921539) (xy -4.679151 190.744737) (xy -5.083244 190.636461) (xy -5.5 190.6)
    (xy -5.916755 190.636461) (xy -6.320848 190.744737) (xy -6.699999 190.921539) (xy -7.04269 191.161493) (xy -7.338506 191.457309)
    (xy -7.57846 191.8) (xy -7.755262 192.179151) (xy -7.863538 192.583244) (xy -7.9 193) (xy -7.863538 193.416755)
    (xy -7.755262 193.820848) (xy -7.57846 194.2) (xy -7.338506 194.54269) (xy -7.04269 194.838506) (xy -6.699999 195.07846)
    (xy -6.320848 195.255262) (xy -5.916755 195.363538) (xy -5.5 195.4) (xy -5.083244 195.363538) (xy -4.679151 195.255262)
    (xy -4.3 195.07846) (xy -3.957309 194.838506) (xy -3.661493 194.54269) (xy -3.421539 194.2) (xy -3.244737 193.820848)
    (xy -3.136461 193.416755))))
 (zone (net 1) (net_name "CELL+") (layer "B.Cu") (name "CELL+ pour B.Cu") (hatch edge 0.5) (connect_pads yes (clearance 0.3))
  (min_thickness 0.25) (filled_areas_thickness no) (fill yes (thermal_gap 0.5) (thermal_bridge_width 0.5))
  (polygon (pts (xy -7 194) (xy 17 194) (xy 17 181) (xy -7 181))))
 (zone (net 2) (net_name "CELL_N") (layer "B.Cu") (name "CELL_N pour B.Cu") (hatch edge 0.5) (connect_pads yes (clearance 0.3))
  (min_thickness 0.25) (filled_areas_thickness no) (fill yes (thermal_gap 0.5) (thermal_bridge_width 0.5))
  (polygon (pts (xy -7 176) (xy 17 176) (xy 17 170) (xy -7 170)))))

